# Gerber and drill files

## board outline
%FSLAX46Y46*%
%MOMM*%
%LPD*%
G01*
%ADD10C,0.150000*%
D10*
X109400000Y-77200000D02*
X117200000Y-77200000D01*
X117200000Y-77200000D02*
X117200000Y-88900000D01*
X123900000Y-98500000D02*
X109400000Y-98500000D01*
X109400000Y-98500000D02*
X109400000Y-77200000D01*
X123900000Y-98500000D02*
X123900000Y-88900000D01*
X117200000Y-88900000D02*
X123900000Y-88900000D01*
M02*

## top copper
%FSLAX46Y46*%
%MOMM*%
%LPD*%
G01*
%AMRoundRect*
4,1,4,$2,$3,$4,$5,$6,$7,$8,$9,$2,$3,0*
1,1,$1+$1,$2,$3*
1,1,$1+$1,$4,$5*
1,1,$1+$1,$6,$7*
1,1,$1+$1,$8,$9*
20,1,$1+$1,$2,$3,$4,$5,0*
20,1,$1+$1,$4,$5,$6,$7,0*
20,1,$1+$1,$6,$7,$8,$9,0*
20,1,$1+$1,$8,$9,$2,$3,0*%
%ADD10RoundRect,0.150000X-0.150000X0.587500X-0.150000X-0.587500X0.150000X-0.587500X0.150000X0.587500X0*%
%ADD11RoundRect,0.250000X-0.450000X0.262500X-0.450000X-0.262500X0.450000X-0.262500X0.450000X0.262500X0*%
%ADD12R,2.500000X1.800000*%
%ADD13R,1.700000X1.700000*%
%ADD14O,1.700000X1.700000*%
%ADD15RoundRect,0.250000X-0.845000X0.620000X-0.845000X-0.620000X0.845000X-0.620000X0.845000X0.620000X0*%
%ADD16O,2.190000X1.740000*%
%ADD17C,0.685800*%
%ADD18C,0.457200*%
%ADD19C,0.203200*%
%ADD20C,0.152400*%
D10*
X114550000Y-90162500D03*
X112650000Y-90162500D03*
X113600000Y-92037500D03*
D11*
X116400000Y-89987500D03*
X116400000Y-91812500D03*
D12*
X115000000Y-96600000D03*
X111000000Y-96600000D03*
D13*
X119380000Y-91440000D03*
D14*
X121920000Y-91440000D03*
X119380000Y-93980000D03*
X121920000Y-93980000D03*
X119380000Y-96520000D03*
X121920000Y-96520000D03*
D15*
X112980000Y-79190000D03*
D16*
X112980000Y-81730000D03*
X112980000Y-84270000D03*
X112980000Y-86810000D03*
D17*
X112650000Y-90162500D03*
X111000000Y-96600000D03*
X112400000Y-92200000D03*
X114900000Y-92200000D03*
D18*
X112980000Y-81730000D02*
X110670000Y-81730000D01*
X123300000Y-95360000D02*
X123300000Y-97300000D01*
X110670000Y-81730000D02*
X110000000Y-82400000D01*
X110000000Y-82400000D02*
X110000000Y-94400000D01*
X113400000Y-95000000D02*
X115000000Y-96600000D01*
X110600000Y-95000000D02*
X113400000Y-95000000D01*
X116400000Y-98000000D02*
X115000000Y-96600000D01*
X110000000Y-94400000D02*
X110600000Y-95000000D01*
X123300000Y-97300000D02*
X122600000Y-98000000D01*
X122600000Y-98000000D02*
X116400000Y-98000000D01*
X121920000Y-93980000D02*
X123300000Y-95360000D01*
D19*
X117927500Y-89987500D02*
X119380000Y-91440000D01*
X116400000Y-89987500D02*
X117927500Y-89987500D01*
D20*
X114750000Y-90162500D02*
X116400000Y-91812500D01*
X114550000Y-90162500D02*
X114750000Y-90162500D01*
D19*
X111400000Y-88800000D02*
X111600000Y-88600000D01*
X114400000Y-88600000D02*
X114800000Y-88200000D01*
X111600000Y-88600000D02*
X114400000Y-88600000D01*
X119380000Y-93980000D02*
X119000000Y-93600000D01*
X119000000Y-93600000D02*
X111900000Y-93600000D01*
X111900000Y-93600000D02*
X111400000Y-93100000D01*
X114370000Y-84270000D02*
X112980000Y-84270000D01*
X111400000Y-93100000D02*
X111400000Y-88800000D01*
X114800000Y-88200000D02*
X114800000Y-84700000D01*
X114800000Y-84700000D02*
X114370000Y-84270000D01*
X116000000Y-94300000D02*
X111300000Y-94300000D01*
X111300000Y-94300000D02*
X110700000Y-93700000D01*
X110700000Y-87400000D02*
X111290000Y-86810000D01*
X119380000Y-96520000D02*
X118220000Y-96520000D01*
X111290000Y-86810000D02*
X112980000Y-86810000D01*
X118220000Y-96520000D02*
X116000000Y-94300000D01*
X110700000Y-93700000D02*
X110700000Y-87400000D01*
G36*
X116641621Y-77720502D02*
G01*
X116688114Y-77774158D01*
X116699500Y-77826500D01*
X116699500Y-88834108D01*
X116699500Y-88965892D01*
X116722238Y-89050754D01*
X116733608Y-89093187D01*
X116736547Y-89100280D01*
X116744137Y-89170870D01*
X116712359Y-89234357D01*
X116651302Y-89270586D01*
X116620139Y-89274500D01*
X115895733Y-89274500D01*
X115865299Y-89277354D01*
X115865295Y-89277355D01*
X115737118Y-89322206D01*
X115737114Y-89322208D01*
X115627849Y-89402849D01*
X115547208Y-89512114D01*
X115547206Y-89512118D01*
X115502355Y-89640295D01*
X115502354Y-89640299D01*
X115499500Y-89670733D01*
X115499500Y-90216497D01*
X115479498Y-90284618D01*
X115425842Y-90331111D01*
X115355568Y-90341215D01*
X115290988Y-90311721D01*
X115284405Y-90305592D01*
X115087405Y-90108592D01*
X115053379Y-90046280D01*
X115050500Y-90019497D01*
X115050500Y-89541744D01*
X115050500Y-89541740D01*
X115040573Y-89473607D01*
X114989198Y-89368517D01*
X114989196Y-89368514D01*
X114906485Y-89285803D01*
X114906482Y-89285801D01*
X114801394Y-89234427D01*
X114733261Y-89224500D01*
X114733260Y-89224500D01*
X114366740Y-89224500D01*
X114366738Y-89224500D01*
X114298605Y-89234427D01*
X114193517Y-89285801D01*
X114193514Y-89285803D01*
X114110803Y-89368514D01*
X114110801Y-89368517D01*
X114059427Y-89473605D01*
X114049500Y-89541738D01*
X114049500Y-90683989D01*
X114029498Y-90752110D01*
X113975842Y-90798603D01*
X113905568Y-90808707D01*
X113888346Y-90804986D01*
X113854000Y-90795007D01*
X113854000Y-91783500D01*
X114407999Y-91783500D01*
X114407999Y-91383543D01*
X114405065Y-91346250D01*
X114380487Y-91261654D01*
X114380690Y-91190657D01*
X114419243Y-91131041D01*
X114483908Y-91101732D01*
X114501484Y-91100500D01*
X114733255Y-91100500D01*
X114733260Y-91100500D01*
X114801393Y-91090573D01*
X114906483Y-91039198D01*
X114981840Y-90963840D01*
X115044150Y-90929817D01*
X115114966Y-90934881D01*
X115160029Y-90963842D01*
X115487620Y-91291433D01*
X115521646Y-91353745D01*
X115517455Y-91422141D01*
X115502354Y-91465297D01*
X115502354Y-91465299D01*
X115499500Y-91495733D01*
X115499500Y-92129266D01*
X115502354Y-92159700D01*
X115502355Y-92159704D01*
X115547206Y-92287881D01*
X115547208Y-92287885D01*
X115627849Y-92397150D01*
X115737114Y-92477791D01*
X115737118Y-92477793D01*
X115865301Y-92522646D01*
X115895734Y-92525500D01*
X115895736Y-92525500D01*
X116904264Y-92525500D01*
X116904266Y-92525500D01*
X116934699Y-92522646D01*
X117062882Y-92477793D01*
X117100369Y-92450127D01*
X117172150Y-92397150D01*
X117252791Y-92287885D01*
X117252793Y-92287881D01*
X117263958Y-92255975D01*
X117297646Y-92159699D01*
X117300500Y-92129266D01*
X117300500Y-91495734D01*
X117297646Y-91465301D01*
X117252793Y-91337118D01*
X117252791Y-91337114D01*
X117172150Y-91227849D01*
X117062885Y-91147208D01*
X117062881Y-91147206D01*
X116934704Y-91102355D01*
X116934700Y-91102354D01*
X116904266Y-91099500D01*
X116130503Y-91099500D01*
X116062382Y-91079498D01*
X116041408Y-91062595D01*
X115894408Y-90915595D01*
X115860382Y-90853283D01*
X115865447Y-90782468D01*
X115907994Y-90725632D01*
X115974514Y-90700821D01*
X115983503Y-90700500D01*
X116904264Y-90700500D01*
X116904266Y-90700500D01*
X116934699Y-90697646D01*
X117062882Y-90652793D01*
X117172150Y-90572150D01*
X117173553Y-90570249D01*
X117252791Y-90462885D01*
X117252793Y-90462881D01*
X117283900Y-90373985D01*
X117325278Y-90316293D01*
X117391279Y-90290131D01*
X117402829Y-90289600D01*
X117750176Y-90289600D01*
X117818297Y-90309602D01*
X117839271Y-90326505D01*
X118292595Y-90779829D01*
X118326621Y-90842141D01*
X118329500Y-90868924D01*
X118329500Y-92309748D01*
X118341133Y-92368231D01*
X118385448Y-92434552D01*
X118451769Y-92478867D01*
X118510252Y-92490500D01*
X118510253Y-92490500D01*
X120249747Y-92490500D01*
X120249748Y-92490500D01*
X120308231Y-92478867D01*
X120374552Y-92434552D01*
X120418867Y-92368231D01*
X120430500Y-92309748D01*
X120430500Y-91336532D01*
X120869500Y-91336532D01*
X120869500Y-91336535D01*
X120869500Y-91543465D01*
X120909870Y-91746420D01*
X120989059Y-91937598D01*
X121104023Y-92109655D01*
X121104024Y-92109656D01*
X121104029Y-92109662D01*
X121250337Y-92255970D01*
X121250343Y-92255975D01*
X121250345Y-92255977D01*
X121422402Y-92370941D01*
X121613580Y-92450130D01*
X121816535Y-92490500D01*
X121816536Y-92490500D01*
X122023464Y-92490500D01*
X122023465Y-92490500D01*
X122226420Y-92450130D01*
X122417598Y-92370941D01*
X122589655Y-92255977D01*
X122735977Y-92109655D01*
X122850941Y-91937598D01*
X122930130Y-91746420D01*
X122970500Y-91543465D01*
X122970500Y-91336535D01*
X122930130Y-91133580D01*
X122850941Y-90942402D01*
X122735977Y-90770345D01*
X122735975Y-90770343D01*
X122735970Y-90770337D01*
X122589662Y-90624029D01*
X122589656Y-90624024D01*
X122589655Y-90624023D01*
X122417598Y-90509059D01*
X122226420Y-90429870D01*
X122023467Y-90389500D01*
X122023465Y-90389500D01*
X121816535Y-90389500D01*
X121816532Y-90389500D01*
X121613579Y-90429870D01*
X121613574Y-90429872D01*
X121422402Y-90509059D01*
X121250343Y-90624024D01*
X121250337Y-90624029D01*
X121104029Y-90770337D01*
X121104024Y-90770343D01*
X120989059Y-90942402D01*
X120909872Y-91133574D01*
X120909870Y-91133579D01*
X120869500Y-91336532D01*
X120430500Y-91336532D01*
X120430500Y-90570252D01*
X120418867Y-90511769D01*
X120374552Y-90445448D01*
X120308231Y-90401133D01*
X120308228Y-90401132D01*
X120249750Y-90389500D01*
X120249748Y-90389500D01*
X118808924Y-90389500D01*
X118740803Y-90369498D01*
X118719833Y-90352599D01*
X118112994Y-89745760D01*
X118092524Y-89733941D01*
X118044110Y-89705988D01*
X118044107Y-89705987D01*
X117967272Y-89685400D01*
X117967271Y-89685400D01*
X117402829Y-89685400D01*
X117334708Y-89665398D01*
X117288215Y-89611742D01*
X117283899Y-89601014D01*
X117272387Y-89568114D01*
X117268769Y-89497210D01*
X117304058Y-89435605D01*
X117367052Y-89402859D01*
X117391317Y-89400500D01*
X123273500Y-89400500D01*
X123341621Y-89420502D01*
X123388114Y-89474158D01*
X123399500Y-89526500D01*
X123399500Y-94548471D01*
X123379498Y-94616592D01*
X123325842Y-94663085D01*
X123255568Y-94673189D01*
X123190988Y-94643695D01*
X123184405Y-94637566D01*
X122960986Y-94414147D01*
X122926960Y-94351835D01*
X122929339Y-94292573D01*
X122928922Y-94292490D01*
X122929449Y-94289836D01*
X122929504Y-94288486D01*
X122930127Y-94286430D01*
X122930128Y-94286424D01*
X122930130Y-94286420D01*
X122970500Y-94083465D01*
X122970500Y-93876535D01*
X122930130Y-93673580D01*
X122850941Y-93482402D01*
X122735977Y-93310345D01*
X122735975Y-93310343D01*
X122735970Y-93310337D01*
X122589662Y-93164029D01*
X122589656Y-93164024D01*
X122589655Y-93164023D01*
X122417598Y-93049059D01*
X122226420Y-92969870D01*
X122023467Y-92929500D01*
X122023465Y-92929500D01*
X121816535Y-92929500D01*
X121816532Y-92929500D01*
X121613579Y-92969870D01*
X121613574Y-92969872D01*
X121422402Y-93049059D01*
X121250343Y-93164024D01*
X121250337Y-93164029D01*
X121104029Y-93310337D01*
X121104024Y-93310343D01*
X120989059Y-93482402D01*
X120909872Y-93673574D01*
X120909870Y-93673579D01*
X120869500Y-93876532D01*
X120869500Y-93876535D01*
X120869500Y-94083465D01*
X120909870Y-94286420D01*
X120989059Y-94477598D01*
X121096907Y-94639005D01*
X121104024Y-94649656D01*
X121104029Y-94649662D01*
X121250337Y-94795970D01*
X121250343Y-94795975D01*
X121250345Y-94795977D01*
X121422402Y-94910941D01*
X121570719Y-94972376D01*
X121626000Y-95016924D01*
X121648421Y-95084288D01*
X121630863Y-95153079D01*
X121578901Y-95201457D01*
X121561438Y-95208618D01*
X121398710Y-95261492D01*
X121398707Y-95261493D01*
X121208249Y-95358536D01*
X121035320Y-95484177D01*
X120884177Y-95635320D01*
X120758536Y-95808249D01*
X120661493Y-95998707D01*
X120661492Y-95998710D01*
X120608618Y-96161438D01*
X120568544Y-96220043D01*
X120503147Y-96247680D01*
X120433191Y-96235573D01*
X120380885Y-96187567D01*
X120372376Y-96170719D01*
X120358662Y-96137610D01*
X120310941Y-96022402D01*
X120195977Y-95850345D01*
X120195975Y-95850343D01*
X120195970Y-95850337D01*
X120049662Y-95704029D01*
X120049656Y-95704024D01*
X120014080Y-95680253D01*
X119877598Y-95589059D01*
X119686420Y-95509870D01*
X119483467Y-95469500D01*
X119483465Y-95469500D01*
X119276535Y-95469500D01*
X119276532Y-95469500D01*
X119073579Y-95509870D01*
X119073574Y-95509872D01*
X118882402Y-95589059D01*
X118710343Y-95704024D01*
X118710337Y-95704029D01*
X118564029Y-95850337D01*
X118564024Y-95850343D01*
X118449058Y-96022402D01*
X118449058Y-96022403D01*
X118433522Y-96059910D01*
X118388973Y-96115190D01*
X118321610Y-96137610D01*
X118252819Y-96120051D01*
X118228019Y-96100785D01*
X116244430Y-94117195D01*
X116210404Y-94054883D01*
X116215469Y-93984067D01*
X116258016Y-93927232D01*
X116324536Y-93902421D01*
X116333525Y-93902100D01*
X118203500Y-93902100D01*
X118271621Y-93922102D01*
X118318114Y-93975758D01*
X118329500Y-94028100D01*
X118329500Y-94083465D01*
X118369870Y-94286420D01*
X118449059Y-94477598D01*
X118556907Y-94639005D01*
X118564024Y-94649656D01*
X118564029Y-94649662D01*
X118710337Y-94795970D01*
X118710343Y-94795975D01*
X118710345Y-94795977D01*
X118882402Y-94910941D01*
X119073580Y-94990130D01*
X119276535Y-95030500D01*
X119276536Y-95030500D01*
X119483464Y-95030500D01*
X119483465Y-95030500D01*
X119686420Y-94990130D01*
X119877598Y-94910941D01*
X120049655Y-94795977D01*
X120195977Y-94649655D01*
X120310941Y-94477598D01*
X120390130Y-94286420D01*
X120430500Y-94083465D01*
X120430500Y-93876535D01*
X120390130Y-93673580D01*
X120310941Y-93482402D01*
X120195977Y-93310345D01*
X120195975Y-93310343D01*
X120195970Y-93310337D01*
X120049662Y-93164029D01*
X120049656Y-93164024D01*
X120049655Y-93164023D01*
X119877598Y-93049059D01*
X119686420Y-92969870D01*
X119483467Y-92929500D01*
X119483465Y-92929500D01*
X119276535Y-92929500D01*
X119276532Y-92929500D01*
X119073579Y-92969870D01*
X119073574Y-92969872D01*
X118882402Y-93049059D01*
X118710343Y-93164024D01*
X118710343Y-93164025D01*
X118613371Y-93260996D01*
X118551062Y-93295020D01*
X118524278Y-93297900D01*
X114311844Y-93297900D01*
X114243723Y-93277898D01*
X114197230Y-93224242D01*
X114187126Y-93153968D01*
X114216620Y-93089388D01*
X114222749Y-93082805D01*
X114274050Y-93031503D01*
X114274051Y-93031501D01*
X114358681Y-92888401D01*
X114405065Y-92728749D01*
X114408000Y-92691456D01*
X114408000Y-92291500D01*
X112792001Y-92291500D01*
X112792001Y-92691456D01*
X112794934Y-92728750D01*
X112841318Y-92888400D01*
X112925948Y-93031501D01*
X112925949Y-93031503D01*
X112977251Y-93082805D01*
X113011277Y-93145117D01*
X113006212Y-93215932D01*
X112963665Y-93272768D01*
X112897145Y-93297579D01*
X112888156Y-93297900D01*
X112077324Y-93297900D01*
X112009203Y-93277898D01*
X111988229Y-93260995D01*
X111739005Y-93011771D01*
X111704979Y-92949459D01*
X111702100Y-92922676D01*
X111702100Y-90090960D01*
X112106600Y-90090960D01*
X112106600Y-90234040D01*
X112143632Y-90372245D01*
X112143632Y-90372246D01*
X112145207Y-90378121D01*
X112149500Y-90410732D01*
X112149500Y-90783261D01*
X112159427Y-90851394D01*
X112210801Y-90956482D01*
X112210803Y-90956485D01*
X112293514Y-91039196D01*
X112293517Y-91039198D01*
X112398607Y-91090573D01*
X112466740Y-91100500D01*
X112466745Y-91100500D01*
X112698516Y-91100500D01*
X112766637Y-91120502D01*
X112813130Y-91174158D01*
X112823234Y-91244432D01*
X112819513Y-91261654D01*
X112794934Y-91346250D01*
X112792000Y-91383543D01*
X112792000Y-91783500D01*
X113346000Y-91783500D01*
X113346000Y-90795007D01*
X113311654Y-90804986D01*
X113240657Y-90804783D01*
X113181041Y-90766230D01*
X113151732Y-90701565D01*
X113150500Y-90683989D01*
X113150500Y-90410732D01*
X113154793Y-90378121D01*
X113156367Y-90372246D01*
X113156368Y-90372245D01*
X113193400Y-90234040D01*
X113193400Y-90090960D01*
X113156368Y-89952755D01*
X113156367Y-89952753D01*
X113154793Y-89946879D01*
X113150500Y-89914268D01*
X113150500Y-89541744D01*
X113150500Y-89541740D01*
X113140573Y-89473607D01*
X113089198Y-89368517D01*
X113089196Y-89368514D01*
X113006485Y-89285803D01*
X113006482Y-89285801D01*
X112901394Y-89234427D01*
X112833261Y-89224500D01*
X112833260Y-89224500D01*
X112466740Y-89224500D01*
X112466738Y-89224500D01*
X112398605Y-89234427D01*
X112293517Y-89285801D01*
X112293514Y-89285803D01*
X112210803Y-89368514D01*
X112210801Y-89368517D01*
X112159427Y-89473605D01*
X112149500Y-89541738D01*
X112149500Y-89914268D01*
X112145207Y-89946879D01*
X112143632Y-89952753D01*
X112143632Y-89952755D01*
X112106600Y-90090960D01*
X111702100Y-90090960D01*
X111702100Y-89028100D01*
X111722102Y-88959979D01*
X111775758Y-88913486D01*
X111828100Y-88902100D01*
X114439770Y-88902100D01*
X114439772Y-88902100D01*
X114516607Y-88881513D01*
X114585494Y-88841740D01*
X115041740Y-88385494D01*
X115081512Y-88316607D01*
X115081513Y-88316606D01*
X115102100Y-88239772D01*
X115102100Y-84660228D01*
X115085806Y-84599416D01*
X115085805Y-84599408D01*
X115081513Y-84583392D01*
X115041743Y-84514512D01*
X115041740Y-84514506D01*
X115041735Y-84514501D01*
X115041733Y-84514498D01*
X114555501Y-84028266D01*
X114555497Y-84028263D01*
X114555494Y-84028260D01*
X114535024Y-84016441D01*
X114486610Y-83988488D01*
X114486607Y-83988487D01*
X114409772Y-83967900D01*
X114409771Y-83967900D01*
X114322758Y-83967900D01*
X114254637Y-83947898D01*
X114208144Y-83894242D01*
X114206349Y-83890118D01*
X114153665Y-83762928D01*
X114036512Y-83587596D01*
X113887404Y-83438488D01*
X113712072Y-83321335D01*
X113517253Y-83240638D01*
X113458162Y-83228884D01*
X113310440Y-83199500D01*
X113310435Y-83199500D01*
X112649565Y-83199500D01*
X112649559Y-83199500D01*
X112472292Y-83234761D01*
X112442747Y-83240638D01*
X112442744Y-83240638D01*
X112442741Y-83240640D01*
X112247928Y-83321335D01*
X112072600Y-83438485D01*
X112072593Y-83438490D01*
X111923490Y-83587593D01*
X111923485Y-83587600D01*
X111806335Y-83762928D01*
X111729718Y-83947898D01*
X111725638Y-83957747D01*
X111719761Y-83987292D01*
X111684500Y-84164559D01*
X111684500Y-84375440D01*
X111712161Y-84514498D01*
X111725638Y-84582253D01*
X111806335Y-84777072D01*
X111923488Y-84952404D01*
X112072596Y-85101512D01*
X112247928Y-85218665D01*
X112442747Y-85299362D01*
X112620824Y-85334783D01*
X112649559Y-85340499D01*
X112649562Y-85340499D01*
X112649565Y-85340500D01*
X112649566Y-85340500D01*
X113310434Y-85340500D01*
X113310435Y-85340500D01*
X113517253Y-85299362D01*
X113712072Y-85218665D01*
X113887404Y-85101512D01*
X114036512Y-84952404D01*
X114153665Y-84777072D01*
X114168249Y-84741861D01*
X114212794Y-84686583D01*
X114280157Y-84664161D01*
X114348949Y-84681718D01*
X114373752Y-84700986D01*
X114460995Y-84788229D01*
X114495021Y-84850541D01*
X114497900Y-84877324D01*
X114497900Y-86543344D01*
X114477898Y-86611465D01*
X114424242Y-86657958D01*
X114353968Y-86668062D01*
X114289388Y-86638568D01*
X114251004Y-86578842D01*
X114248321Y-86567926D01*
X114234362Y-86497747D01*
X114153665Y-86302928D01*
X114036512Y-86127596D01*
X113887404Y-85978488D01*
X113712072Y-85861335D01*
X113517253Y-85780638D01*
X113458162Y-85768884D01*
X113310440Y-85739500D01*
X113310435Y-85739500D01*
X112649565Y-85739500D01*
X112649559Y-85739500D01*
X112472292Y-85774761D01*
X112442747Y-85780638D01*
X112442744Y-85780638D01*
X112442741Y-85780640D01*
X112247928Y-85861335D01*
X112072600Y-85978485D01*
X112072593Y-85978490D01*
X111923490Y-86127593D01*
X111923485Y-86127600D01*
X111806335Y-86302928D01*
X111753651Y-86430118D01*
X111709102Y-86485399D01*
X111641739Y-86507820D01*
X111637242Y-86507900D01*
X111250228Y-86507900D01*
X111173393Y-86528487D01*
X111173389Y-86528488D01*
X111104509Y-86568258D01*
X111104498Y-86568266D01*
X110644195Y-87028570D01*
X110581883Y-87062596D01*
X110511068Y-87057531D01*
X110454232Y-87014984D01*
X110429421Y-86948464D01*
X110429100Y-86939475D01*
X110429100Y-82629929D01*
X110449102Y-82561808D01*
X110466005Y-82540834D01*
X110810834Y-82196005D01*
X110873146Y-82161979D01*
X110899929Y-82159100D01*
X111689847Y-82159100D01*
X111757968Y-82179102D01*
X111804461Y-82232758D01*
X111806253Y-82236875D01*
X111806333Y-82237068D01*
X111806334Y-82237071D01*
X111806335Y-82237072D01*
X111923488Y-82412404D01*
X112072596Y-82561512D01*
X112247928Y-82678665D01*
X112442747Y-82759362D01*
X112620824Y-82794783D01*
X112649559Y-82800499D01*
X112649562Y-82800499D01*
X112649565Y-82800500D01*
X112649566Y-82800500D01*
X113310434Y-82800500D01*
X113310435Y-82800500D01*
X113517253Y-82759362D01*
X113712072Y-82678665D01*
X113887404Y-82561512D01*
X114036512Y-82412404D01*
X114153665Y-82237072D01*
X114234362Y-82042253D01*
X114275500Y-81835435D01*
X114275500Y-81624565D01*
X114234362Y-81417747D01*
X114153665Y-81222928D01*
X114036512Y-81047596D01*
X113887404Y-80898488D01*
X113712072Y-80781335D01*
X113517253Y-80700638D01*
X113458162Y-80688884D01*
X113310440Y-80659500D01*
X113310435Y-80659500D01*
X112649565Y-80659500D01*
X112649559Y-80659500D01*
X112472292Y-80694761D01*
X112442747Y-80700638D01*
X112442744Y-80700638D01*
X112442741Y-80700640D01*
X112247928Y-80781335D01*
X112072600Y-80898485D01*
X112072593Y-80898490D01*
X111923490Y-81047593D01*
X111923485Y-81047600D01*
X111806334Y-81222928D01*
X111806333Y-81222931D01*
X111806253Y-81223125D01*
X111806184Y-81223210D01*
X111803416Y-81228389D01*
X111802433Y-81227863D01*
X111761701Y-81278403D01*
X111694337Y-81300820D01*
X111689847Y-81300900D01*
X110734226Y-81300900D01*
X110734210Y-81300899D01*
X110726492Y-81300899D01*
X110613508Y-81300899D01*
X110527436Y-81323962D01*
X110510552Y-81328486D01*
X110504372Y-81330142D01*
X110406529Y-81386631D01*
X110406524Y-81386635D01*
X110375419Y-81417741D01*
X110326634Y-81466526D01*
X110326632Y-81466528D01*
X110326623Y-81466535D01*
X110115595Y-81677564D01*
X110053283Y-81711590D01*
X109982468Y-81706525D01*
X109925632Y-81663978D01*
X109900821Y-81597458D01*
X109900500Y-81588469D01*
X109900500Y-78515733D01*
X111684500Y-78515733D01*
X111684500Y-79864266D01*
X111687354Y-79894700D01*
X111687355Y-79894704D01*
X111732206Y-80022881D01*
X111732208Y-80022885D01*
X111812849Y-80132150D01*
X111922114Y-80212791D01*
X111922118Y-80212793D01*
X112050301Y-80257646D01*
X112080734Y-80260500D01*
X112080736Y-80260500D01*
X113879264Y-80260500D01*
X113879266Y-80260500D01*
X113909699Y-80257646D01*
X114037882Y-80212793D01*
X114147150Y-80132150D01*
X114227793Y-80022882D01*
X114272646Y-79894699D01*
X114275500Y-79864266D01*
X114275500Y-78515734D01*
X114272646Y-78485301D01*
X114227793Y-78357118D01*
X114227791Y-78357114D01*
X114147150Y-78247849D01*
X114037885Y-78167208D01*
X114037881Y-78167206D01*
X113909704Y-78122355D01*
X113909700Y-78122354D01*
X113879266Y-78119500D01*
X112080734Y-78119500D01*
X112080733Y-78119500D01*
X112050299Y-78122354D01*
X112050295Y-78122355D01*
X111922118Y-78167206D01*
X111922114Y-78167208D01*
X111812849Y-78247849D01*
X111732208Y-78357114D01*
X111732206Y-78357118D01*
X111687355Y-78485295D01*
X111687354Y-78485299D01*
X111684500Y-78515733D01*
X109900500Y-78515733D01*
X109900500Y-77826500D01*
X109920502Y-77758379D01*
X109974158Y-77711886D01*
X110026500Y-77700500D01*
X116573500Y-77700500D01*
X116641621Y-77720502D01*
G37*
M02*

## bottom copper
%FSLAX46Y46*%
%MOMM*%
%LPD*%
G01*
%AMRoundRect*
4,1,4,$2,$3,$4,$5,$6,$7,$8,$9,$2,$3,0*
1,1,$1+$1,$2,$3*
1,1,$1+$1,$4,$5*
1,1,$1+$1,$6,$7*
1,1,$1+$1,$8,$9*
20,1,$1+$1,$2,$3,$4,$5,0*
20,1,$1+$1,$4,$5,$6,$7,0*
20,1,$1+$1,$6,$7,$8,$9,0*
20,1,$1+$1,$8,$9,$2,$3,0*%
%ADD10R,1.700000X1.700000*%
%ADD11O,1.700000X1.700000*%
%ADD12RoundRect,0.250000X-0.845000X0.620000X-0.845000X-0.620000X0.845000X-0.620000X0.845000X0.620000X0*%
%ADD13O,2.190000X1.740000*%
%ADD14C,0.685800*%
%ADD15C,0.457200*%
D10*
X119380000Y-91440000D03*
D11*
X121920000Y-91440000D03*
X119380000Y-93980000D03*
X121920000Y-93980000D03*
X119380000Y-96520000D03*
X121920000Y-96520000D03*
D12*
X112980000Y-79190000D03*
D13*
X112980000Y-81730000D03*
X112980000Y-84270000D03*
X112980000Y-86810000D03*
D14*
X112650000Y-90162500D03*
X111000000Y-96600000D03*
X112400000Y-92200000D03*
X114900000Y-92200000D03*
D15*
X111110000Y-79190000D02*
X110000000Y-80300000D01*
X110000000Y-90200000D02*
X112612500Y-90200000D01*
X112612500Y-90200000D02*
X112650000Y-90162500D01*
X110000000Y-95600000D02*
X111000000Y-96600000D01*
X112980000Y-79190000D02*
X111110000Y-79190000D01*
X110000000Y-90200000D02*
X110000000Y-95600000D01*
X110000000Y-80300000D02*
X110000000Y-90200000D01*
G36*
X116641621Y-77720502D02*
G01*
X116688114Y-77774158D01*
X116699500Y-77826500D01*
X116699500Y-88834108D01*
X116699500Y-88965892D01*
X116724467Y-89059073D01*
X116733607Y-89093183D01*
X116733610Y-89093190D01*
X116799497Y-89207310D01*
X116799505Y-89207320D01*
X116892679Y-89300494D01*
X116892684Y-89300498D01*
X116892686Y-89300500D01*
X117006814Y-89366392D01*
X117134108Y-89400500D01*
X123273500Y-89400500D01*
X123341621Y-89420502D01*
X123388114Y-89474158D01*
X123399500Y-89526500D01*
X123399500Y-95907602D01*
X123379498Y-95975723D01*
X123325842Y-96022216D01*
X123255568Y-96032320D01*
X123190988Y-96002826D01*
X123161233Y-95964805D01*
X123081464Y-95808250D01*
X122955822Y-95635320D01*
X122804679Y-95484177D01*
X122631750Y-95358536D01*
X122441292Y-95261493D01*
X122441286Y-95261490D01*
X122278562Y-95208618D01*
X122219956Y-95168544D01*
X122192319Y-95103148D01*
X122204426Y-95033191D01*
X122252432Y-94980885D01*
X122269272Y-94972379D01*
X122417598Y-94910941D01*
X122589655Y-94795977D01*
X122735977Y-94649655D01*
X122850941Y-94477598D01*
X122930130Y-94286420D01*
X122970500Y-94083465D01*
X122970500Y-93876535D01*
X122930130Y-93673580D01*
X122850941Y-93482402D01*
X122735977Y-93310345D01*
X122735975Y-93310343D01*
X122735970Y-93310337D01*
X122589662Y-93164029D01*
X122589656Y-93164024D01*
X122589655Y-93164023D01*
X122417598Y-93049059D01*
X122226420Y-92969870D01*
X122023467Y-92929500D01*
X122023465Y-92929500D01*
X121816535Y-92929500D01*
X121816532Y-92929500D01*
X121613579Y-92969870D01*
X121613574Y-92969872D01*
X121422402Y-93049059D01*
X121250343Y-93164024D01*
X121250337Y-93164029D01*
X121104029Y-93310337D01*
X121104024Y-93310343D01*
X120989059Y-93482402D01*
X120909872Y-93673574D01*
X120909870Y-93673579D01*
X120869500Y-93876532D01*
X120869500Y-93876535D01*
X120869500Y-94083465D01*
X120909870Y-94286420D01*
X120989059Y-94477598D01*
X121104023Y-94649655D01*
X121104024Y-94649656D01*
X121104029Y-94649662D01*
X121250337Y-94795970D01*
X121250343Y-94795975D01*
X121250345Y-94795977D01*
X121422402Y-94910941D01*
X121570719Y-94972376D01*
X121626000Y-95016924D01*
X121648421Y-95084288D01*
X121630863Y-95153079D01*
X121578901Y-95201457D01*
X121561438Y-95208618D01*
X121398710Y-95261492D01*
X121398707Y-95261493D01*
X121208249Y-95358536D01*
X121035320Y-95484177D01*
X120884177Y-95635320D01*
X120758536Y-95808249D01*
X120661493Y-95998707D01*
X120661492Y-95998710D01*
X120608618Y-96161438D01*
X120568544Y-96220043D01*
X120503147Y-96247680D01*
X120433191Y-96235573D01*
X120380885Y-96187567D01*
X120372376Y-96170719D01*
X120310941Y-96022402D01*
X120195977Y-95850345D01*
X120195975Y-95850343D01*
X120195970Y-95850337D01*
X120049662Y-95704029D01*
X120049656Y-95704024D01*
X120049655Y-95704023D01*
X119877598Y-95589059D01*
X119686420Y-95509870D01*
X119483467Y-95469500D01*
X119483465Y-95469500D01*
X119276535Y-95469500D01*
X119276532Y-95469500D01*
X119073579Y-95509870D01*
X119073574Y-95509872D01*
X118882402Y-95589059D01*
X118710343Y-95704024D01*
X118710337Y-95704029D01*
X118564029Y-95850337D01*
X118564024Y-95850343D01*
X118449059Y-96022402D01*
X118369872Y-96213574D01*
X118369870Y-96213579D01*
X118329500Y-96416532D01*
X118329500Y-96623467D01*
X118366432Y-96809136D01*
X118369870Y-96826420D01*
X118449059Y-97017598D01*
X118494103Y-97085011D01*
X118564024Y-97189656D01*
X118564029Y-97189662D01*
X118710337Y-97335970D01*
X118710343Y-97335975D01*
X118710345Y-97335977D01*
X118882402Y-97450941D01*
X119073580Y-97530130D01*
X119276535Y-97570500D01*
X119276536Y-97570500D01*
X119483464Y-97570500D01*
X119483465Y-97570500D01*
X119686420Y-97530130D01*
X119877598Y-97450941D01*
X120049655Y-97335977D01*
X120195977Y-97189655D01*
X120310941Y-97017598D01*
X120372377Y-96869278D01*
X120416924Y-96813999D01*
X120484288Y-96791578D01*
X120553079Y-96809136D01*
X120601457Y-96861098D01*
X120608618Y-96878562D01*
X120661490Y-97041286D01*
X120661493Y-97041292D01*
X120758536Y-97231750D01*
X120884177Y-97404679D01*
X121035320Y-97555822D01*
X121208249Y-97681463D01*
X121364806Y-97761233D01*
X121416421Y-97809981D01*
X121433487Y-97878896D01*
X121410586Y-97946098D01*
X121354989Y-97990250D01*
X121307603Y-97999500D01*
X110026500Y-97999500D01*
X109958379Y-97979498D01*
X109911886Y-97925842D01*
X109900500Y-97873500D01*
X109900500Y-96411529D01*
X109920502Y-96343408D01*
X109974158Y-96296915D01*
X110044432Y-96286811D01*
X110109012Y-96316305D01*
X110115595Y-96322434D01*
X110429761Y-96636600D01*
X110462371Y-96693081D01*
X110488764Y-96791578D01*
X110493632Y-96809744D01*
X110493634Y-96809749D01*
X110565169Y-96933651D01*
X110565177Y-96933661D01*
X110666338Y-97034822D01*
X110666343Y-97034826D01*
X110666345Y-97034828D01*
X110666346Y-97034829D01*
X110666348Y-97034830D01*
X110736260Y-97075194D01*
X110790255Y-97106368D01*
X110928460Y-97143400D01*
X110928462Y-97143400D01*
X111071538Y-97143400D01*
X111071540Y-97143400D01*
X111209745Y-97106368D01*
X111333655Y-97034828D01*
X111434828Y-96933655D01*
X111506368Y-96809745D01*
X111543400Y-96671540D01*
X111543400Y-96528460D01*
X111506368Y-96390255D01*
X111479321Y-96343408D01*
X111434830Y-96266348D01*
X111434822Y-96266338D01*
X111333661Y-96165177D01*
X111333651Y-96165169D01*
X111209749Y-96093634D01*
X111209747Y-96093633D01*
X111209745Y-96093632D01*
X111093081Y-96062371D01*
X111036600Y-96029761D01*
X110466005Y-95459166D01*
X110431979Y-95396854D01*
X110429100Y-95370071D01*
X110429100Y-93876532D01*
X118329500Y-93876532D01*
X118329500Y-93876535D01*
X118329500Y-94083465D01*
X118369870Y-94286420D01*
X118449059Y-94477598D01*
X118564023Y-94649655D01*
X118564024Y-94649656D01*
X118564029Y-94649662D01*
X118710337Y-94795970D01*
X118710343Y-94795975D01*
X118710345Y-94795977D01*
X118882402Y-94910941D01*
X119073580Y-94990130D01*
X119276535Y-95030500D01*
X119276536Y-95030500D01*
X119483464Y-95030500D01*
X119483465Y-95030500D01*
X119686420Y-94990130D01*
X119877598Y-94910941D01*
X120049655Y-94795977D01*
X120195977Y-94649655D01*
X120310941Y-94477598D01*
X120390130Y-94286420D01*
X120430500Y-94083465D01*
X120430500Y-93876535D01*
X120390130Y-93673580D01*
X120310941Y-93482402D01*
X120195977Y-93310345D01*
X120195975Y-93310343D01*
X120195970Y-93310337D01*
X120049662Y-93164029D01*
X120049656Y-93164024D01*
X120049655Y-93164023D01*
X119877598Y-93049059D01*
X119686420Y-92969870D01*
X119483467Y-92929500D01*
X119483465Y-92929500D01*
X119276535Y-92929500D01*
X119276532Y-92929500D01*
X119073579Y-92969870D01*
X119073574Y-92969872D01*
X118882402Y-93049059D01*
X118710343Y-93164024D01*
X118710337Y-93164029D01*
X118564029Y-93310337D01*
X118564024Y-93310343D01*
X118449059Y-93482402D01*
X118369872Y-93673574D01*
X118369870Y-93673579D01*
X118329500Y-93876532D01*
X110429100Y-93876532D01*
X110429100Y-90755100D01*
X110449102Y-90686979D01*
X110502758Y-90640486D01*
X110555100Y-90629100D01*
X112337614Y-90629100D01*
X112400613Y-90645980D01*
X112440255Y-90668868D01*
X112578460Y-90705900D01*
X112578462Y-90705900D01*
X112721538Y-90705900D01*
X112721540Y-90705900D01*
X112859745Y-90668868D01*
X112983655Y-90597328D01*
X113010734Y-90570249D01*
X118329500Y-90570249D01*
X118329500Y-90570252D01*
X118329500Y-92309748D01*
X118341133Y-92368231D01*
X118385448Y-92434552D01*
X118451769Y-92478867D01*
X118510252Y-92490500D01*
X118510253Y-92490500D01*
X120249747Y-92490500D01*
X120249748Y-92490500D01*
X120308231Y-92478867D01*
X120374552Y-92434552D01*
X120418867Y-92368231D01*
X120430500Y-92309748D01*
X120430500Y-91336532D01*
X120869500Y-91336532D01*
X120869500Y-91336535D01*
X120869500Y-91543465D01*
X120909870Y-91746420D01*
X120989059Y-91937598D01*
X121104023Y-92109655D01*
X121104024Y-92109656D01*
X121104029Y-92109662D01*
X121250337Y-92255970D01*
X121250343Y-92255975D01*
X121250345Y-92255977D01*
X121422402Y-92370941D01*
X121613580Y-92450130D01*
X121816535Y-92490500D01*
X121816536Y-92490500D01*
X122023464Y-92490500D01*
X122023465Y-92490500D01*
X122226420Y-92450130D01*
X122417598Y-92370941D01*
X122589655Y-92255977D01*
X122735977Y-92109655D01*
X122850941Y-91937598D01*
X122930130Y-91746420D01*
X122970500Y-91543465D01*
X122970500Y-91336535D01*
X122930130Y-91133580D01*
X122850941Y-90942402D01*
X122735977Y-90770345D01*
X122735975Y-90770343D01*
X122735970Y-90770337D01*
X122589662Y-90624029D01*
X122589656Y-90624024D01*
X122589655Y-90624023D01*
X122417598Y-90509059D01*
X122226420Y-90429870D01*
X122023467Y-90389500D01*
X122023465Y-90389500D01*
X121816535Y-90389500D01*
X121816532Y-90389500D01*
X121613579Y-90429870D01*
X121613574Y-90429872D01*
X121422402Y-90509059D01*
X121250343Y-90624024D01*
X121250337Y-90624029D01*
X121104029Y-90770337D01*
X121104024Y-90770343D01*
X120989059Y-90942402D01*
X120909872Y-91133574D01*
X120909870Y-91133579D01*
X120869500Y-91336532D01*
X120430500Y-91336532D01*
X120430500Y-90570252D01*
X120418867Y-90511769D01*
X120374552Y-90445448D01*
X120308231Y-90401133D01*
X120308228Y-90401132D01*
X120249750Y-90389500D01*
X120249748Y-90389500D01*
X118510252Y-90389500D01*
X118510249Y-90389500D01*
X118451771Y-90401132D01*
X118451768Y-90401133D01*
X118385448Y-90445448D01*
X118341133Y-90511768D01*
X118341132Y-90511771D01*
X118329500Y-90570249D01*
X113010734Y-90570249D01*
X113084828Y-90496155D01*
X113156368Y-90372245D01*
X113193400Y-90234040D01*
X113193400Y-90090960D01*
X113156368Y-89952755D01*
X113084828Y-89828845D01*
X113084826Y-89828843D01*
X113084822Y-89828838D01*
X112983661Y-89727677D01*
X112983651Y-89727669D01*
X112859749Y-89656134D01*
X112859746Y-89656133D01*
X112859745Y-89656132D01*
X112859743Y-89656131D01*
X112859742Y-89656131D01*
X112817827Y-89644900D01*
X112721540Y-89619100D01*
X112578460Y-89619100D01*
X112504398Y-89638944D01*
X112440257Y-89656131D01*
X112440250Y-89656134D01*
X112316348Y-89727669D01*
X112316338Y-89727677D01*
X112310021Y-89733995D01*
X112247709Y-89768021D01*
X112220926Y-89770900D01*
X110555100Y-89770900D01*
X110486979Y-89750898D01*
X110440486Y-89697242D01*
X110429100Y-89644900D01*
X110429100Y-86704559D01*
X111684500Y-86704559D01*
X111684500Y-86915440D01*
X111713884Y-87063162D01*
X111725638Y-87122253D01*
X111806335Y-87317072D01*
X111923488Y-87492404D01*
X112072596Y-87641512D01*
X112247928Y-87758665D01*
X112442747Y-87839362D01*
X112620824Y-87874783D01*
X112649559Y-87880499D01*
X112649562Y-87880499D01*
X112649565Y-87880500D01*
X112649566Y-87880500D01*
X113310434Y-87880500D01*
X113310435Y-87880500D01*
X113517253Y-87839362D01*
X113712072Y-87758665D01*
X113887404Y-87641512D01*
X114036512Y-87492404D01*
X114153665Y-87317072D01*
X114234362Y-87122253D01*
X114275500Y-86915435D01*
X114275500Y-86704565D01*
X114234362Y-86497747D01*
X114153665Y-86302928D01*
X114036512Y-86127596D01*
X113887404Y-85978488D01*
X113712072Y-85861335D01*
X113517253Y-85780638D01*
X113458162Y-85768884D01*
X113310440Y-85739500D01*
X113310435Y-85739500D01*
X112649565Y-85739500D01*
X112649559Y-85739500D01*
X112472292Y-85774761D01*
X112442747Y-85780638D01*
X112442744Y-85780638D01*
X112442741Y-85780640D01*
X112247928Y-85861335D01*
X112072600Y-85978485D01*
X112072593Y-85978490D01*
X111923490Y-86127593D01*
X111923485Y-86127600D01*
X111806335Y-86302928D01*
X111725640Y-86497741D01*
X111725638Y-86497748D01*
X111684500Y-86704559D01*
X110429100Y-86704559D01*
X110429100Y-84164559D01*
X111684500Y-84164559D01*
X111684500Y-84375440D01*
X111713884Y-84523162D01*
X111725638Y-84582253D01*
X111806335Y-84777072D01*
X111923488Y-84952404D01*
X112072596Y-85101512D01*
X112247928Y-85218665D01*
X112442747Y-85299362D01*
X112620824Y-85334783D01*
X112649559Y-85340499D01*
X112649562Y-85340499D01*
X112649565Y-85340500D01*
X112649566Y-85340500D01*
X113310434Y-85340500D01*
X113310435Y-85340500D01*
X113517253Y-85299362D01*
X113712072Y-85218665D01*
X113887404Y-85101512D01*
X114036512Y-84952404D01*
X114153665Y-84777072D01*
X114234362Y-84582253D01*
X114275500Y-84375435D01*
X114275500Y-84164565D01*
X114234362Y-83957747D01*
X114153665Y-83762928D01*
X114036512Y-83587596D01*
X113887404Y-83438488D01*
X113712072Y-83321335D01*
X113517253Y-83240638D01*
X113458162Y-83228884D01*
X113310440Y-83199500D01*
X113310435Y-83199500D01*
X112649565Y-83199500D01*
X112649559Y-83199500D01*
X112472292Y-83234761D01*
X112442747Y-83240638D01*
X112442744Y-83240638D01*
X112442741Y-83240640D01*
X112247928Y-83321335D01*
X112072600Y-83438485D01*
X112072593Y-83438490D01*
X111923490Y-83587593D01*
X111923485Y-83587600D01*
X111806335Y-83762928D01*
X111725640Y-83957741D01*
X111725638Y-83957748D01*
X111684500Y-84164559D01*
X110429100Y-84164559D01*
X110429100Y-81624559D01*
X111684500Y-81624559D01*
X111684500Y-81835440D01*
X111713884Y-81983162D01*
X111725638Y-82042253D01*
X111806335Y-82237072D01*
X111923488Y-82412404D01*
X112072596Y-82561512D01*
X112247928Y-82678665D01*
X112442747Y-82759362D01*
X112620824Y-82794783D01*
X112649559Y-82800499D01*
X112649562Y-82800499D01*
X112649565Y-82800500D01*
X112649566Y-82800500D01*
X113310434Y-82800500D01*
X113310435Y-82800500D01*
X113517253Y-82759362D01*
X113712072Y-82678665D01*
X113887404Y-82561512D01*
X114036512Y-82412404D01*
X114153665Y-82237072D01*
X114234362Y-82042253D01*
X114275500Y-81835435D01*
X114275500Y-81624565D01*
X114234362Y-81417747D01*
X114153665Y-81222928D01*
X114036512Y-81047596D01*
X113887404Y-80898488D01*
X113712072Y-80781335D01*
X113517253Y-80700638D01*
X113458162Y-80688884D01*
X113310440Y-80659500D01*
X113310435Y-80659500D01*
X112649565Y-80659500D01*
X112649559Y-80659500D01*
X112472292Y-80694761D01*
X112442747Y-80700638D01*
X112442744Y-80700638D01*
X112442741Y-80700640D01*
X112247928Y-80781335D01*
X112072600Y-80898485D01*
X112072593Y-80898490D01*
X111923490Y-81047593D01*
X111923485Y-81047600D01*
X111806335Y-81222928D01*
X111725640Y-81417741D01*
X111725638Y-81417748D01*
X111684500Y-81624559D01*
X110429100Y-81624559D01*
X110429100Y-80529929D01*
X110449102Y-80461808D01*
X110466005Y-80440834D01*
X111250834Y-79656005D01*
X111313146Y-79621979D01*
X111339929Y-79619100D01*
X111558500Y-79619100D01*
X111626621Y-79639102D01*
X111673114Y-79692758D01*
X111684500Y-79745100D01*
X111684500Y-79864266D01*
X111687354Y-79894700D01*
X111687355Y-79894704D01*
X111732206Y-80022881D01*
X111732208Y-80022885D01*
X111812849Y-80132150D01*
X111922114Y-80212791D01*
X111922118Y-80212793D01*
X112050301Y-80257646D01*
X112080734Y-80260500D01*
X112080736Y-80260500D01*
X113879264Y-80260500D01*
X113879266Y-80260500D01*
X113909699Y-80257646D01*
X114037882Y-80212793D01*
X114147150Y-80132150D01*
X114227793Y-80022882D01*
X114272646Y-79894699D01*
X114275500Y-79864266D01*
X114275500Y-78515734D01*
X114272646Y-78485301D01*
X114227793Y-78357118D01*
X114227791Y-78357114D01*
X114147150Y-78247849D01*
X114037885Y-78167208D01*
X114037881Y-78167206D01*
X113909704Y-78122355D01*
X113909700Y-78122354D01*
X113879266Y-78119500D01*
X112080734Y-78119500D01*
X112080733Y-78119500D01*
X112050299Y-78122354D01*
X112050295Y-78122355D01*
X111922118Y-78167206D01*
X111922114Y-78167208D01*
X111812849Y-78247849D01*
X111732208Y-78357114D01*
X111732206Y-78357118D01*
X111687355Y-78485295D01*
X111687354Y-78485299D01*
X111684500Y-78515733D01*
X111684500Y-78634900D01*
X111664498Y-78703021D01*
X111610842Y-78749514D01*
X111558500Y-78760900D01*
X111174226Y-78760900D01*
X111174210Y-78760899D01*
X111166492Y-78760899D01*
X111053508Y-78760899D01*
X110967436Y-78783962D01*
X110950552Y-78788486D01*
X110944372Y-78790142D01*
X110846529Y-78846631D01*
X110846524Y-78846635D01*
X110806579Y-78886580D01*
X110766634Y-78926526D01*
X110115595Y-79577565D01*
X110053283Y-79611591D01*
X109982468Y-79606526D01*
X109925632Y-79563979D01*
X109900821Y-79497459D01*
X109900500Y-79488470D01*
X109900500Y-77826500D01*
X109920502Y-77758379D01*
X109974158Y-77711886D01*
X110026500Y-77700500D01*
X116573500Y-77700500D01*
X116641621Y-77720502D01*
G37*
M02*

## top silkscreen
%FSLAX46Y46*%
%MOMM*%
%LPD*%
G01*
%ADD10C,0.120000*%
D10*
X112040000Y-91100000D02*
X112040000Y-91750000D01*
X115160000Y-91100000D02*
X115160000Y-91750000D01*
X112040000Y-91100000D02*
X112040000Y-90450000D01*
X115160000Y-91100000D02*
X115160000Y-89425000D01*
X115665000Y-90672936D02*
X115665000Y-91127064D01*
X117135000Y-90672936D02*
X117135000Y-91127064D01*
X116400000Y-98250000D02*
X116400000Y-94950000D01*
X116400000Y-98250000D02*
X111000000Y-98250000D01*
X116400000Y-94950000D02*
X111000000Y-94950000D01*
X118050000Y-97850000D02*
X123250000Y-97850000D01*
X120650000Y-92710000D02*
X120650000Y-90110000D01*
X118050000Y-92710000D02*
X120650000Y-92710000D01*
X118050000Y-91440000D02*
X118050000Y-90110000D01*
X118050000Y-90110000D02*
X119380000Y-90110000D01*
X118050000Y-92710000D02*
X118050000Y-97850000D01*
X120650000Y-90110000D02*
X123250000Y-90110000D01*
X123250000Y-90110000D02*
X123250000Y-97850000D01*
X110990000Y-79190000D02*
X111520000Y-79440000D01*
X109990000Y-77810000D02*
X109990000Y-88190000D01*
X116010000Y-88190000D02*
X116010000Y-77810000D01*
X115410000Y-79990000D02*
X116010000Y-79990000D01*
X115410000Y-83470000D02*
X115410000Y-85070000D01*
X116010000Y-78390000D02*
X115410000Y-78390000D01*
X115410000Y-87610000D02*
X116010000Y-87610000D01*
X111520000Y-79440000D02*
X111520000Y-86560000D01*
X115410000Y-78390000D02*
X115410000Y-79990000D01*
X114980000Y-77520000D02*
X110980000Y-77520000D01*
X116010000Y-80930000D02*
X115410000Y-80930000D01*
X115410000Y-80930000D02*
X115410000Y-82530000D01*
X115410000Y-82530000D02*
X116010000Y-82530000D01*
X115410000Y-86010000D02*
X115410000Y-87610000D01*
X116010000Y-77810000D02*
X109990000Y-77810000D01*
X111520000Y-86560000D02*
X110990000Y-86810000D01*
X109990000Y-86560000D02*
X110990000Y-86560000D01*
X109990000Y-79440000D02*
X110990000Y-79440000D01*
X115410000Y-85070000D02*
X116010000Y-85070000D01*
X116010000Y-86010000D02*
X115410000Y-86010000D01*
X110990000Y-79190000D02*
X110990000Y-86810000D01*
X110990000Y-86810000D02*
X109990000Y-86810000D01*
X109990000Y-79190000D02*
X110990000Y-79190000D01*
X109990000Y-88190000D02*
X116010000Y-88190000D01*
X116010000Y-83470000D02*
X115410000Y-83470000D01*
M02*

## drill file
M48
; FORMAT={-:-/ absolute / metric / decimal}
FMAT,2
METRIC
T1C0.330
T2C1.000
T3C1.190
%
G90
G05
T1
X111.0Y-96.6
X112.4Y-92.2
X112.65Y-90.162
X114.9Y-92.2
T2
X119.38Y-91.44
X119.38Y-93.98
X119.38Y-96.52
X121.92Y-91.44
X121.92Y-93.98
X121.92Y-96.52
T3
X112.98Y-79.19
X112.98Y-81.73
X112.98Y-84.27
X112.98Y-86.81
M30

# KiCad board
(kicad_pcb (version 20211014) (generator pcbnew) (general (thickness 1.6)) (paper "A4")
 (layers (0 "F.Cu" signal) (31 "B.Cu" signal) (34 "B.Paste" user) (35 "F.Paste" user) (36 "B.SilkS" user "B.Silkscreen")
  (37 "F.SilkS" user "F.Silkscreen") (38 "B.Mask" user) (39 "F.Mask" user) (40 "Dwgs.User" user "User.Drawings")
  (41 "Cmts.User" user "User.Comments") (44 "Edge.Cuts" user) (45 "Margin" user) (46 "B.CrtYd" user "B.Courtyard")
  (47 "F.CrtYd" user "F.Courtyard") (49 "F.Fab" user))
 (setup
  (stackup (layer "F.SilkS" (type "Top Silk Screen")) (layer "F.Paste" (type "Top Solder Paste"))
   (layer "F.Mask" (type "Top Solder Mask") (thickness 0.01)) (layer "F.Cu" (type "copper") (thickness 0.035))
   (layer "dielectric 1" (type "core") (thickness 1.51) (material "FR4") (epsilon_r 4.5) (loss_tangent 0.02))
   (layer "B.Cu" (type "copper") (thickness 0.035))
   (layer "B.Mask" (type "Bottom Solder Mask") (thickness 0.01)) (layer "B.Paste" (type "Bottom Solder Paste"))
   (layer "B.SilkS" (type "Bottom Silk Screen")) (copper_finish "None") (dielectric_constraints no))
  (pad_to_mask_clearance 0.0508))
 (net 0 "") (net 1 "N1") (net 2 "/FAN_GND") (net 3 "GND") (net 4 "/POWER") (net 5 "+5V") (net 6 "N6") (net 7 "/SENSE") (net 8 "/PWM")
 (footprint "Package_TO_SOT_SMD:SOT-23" (layer "F.Cu") (at 113.6 91.1 -90)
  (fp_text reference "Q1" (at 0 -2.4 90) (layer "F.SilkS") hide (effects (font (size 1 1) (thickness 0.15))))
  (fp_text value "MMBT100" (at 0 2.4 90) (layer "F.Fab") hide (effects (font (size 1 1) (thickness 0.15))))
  (fp_line (start 0 1.56) (end 0.65 1.56) (layer "F.SilkS") (width 0.12))
  (fp_line (start 0 -1.56) (end 0.65 -1.56) (layer "F.SilkS") (width 0.12))
  (fp_line (start 0 1.56) (end -0.65 1.56) (layer "F.SilkS") (width 0.12))
  (fp_line (start 0 -1.56) (end -1.675 -1.56) (layer "F.SilkS") (width 0.12))
  (pad "1" smd roundrect (at -0.9375 -0.95 270) (size 1.475 0.6) (layers "F.Cu" "F.Paste" "F.Mask") (roundrect_rratio 0.25) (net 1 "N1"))
  (pad "2" smd roundrect (at -0.9375 0.95 270) (size 1.475 0.6) (layers "F.Cu" "F.Paste" "F.Mask") (roundrect_rratio 0.25)
   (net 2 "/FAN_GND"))
  (pad "3" smd roundrect (at 0.9375 0 270) (size 1.475 0.6) (layers "F.Cu" "F.Paste" "F.Mask") (roundrect_rratio 0.25) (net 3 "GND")))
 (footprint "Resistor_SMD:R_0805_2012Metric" (layer "F.Cu") (at 116.4 90.9 -90)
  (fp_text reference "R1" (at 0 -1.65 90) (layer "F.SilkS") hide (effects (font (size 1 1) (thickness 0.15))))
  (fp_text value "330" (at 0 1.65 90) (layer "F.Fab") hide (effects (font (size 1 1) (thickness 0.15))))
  (fp_line (start -0.227064 0.735) (end 0.227064 0.735) (layer "F.SilkS") (width 0.12))
  (fp_line (start -0.227064 -0.735) (end 0.227064 -0.735) (layer "F.SilkS") (width 0.12))
  (pad "1" smd roundrect (at -0.9125 0 270) (size 1.025 1.4) (layers "F.Cu" "F.Paste" "F.Mask") (roundrect_rratio 0.243902439)
   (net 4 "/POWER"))
  (pad "2" smd roundrect (at 0.9125 0 270) (size 1.025 1.4) (layers "F.Cu" "F.Paste" "F.Mask") (roundrect_rratio 0.243902439) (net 1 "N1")))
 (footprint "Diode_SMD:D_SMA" (layer "F.Cu") (at 113 96.6 180)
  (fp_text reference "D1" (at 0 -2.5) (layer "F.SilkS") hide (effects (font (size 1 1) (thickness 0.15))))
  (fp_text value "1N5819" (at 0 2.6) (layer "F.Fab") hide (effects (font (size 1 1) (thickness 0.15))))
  (fp_line (start -3.4 -1.65) (end -3.4 1.65) (layer "F.SilkS") (width 0.12))
  (fp_line (start -3.4 -1.65) (end 2 -1.65) (layer "F.SilkS") (width 0.12))
  (fp_line (start -3.4 1.65) (end 2 1.65) (layer "F.SilkS") (width 0.12))
  (pad "1" smd rect (at -2 0 180) (size 2.5 1.8) (layers "F.Cu" "F.Paste" "F.Mask") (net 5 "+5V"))
  (pad "2" smd rect (at 2 0 180) (size 2.5 1.8) (layers "F.Cu" "F.Paste" "F.Mask") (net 2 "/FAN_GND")))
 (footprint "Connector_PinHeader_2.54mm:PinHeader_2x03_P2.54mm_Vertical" (layer "F.Cu") (at 119.38 91.44)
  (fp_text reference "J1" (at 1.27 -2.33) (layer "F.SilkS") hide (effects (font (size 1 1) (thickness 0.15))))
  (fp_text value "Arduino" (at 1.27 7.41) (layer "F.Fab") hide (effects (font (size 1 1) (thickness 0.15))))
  (fp_line (start -1.33 6.41) (end 3.87 6.41) (layer "F.SilkS") (width 0.12))
  (fp_line (start 1.27 1.27) (end 1.27 -1.33) (layer "F.SilkS") (width 0.12))
  (fp_line (start -1.33 1.27) (end 1.27 1.27) (layer "F.SilkS") (width 0.12))
  (fp_line (start -1.33 0) (end -1.33 -1.33) (layer "F.SilkS") (width 0.12))
  (fp_line (start -1.33 -1.33) (end 0 -1.33) (layer "F.SilkS") (width 0.12))
  (fp_line (start -1.33 1.27) (end -1.33 6.41) (layer "F.SilkS") (width 0.12))
  (fp_line (start 1.27 -1.33) (end 3.87 -1.33) (layer "F.SilkS") (width 0.12))
  (fp_line (start 3.87 -1.33) (end 3.87 6.41) (layer "F.SilkS") (width 0.12))
  (pad "1" thru_hole rect (at 0 0) (size 1.7 1.7) (drill 1) (layers *.Cu *.Mask) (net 4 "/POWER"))
  (pad "2" thru_hole oval (at 2.54 0) (size 1.7 1.7) (drill 1) (layers *.Cu *.Mask) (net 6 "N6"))
  (pad "3" thru_hole oval (at 0 2.54) (size 1.7 1.7) (drill 1) (layers *.Cu *.Mask) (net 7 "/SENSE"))
  (pad "4" thru_hole oval (at 2.54 2.54) (size 1.7 1.7) (drill 1) (layers *.Cu *.Mask) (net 5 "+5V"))
  (pad "5" thru_hole oval (at 0 5.08) (size 1.7 1.7) (drill 1) (layers *.Cu *.Mask) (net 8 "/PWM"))
  (pad "6" thru_hole oval (at 2.54 5.08) (size 1.7 1.7) (drill 1) (layers *.Cu *.Mask) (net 3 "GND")))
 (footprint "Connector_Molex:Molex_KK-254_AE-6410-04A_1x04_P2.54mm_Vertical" (layer "F.Cu") (at 112.98 79.19 -90)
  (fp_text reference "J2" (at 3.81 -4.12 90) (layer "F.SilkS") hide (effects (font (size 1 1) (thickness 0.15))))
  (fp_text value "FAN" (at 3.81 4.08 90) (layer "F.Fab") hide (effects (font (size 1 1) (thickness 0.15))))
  (fp_line (start 0 1.99) (end 0.25 1.46) (layer "F.SilkS") (width 0.12))
  (fp_line (start -1.38 2.99) (end 9 2.99) (layer "F.SilkS") (width 0.12))
  (fp_line (start 9 -3.03) (end -1.38 -3.03) (layer "F.SilkS") (width 0.12))
  (fp_line (start 0.8 -2.43) (end 0.8 -3.03) (layer "F.SilkS") (width 0.12))
  (fp_line (start 4.28 -2.43) (end 5.88 -2.43) (layer "F.SilkS") (width 0.12))
  (fp_line (start -0.8 -3.03) (end -0.8 -2.43) (layer "F.SilkS") (width 0.12))
  (fp_line (start 8.42 -2.43) (end 8.42 -3.03) (layer "F.SilkS") (width 0.12))
  (fp_line (start 0.25 1.46) (end 7.37 1.46) (layer "F.SilkS") (width 0.12))
  (fp_line (start -0.8 -2.43) (end 0.8 -2.43) (layer "F.SilkS") (width 0.12))
  (fp_line (start -1.67 -2) (end -1.67 2) (layer "F.SilkS") (width 0.12))
  (fp_line (start 1.74 -3.03) (end 1.74 -2.43) (layer "F.SilkS") (width 0.12))
  (fp_line (start 1.74 -2.43) (end 3.34 -2.43) (layer "F.SilkS") (width 0.12))
  (fp_line (start 3.34 -2.43) (end 3.34 -3.03) (layer "F.SilkS") (width 0.12))
  (fp_line (start 6.82 -2.43) (end 8.42 -2.43) (layer "F.SilkS") (width 0.12))
  (fp_line (start -1.38 -3.03) (end -1.38 2.99) (layer "F.SilkS") (width 0.12))
  (fp_line (start 7.37 1.46) (end 7.62 1.99) (layer "F.SilkS") (width 0.12))
  (fp_line (start 7.37 2.99) (end 7.37 1.99) (layer "F.SilkS") (width 0.12))
  (fp_line (start 0.25 2.99) (end 0.25 1.99) (layer "F.SilkS") (width 0.12))
  (fp_line (start 5.88 -2.43) (end 5.88 -3.03) (layer "F.SilkS") (width 0.12))
  (fp_line (start 6.82 -3.03) (end 6.82 -2.43) (layer "F.SilkS") (width 0.12))
  (fp_line (start 0 1.99) (end 7.62 1.99) (layer "F.SilkS") (width 0.12))
  (fp_line (start 7.62 1.99) (end 7.62 2.99) (layer "F.SilkS") (width 0.12))
  (fp_line (start 0 2.99) (end 0 1.99) (layer "F.SilkS") (width 0.12))
  (fp_line (start 9 2.99) (end 9 -3.03) (layer "F.SilkS") (width 0.12))
  (fp_line (start 4.28 -3.03) (end 4.28 -2.43) (layer "F.SilkS") (width 0.12))
  (pad "1" thru_hole roundrect (at 0 0 270) (size 1.74 2.19) (drill 1.19) (layers *.Cu *.Mask) (roundrect_rratio 0.1436781609)
   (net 2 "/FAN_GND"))
  (pad "2" thru_hole oval (at 2.54 0 270) (size 1.74 2.19) (drill 1.19) (layers *.Cu *.Mask) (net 5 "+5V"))
  (pad "3" thru_hole oval (at 5.08 0 270) (size 1.74 2.19) (drill 1.19) (layers *.Cu *.Mask) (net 7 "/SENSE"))
  (pad "4" thru_hole oval (at 7.62 0 270) (size 1.74 2.19) (drill 1.19) (layers *.Cu *.Mask) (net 8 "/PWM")))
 (gr_line (start 109.4 77.2) (end 117.2 77.2) (layer "Edge.Cuts") (width 0.15))
 (gr_line (start 117.2 77.2) (end 117.2 88.9) (layer "Edge.Cuts") (width 0.15))
 (gr_line (start 123.9 98.5) (end 109.4 98.5) (layer "Edge.Cuts") (width 0.15))
 (gr_line (start 109.4 98.5) (end 109.4 77.2) (layer "Edge.Cuts") (width 0.15))
 (gr_line (start 123.9 98.5) (end 123.9 88.9) (layer "Edge.Cuts") (width 0.15))
 (gr_line (start 117.2 88.9) (end 123.9 88.9) (layer "Edge.Cuts") (width 0.15))
 (segment (start 112.98 81.73) (end 110.67 81.73) (width 0.4572) (layer "F.Cu") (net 5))
 (segment (start 123.3 95.36) (end 123.3 97.3) (width 0.4572) (layer "F.Cu") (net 5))
 (segment (start 110.67 81.73) (end 110 82.4) (width 0.4572) (layer "F.Cu") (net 5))
 (segment (start 110 82.4) (end 110 94.4) (width 0.4572) (layer "F.Cu") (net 5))
 (segment (start 113.4 95) (end 115 96.6) (width 0.4572) (layer "F.Cu") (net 5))
 (segment (start 110.6 95) (end 113.4 95) (width 0.4572) (layer "F.Cu") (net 5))
 (segment (start 116.4 98) (end 115 96.6) (width 0.4572) (layer "F.Cu") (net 5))
 (segment (start 110 94.4) (end 110.6 95) (width 0.4572) (layer "F.Cu") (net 5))
 (segment (start 123.3 97.3) (end 122.6 98) (width 0.4572) (layer "F.Cu") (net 5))
 (segment (start 122.6 98) (end 116.4 98) (width 0.4572) (layer "F.Cu") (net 5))
 (segment (start 121.92 93.98) (end 123.3 95.36) (width 0.4572) (layer "F.Cu") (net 5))
 (via (at 112.65 90.1625) (size 0.6858) (drill 0.3302) (layers "F.Cu" "B.Cu") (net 2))
 (via (at 111 96.6) (size 0.6858) (drill 0.3302) (layers "F.Cu" "B.Cu") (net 2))
 (segment (start 111.11 79.19) (end 110 80.3) (width 0.4572) (layer "B.Cu") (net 2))
 (segment (start 110 90.2) (end 112.6125 90.2) (width 0.4572) (layer "B.Cu") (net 2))
 (segment (start 112.6125 90.2) (end 112.65 90.1625) (width 0.4572) (layer "B.Cu") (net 2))
 (segment (start 110 95.6) (end 111 96.6) (width 0.4572) (layer "B.Cu") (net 2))
 (segment (start 112.98 79.19) (end 111.11 79.19) (width 0.4572) (layer "B.Cu") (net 2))
 (segment (start 110 90.2) (end 110 95.6) (width 0.4572) (layer "B.Cu") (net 2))
 (segment (start 110 80.3) (end 110 90.2) (width 0.4572) (layer "B.Cu") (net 2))
 (segment (start 117.9275 89.9875) (end 119.38 91.44) (width 0.2032) (layer "F.Cu") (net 4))
 (segment (start 116.4 89.9875) (end 117.9275 89.9875) (width 0.2032) (layer "F.Cu") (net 4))
 (segment (start 114.75 90.1625) (end 116.4 91.8125) (width 0.1524) (layer "F.Cu") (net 1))
 (segment (start 114.55 90.1625) (end 114.75 90.1625) (width 0.1524) (layer "F.Cu") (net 1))
 (segment (start 111.4 88.8) (end 111.6 88.6) (width 0.2032) (layer "F.Cu") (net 7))
 (segment (start 114.4 88.6) (end 114.8 88.2) (width 0.2032) (layer "F.Cu") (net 7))
 (segment (start 111.6 88.6) (end 114.4 88.6) (width 0.2032) (layer "F.Cu") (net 7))
 (segment (start 119.38 93.98) (end 119 93.6) (width 0.2032) (layer "F.Cu") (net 7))
 (segment (start 119 93.6) (end 111.9 93.6) (width 0.2032) (layer "F.Cu") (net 7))
 (segment (start 111.9 93.6) (end 111.4 93.1) (width 0.2032) (layer "F.Cu") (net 7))
 (segment (start 114.37 84.27) (end 112.98 84.27) (width 0.2032) (layer "F.Cu") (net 7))
 (segment (start 111.4 93.1) (end 111.4 88.8) (width 0.2032) (layer "F.Cu") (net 7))
 (segment (start 114.8 88.2) (end 114.8 84.7) (width 0.2032) (layer "F.Cu") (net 7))
 (segment (start 114.8 84.7) (end 114.37 84.27) (width 0.2032) (layer "F.Cu") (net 7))
 (segment (start 116 94.3) (end 111.3 94.3) (width 0.2032) (layer "F.Cu") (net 8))
 (segment (start 111.3 94.3) (end 110.7 93.7) (width 0.2032) (layer "F.Cu") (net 8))
 (segment (start 110.7 87.4) (end 111.29 86.81) (width 0.2032) (layer "F.Cu") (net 8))
 (segment (start 119.38 96.52) (end 118.22 96.52) (width 0.2032) (layer "F.Cu") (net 8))
 (segment (start 111.29 86.81) (end 112.98 86.81) (width 0.2032) (layer "F.Cu") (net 8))
 (segment (start 118.22 96.52) (end 116 94.3) (width 0.2032) (layer "F.Cu") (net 8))
 (segment (start 110.7 93.7) (end 110.7 87.4) (width 0.2032) (layer "F.Cu") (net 8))
 (via (at 112.4 92.2) (size 0.6858) (drill 0.3302) (layers "F.Cu" "B.Cu") (free) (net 3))
 (via (at 114.9 92.2) (size 0.6858) (drill 0.3302) (layers "F.Cu" "B.Cu") (free) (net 3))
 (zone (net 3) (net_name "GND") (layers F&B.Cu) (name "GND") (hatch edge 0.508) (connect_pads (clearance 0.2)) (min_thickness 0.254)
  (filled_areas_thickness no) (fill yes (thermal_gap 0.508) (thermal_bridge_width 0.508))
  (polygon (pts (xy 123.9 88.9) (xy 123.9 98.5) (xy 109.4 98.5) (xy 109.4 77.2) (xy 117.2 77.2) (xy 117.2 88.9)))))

